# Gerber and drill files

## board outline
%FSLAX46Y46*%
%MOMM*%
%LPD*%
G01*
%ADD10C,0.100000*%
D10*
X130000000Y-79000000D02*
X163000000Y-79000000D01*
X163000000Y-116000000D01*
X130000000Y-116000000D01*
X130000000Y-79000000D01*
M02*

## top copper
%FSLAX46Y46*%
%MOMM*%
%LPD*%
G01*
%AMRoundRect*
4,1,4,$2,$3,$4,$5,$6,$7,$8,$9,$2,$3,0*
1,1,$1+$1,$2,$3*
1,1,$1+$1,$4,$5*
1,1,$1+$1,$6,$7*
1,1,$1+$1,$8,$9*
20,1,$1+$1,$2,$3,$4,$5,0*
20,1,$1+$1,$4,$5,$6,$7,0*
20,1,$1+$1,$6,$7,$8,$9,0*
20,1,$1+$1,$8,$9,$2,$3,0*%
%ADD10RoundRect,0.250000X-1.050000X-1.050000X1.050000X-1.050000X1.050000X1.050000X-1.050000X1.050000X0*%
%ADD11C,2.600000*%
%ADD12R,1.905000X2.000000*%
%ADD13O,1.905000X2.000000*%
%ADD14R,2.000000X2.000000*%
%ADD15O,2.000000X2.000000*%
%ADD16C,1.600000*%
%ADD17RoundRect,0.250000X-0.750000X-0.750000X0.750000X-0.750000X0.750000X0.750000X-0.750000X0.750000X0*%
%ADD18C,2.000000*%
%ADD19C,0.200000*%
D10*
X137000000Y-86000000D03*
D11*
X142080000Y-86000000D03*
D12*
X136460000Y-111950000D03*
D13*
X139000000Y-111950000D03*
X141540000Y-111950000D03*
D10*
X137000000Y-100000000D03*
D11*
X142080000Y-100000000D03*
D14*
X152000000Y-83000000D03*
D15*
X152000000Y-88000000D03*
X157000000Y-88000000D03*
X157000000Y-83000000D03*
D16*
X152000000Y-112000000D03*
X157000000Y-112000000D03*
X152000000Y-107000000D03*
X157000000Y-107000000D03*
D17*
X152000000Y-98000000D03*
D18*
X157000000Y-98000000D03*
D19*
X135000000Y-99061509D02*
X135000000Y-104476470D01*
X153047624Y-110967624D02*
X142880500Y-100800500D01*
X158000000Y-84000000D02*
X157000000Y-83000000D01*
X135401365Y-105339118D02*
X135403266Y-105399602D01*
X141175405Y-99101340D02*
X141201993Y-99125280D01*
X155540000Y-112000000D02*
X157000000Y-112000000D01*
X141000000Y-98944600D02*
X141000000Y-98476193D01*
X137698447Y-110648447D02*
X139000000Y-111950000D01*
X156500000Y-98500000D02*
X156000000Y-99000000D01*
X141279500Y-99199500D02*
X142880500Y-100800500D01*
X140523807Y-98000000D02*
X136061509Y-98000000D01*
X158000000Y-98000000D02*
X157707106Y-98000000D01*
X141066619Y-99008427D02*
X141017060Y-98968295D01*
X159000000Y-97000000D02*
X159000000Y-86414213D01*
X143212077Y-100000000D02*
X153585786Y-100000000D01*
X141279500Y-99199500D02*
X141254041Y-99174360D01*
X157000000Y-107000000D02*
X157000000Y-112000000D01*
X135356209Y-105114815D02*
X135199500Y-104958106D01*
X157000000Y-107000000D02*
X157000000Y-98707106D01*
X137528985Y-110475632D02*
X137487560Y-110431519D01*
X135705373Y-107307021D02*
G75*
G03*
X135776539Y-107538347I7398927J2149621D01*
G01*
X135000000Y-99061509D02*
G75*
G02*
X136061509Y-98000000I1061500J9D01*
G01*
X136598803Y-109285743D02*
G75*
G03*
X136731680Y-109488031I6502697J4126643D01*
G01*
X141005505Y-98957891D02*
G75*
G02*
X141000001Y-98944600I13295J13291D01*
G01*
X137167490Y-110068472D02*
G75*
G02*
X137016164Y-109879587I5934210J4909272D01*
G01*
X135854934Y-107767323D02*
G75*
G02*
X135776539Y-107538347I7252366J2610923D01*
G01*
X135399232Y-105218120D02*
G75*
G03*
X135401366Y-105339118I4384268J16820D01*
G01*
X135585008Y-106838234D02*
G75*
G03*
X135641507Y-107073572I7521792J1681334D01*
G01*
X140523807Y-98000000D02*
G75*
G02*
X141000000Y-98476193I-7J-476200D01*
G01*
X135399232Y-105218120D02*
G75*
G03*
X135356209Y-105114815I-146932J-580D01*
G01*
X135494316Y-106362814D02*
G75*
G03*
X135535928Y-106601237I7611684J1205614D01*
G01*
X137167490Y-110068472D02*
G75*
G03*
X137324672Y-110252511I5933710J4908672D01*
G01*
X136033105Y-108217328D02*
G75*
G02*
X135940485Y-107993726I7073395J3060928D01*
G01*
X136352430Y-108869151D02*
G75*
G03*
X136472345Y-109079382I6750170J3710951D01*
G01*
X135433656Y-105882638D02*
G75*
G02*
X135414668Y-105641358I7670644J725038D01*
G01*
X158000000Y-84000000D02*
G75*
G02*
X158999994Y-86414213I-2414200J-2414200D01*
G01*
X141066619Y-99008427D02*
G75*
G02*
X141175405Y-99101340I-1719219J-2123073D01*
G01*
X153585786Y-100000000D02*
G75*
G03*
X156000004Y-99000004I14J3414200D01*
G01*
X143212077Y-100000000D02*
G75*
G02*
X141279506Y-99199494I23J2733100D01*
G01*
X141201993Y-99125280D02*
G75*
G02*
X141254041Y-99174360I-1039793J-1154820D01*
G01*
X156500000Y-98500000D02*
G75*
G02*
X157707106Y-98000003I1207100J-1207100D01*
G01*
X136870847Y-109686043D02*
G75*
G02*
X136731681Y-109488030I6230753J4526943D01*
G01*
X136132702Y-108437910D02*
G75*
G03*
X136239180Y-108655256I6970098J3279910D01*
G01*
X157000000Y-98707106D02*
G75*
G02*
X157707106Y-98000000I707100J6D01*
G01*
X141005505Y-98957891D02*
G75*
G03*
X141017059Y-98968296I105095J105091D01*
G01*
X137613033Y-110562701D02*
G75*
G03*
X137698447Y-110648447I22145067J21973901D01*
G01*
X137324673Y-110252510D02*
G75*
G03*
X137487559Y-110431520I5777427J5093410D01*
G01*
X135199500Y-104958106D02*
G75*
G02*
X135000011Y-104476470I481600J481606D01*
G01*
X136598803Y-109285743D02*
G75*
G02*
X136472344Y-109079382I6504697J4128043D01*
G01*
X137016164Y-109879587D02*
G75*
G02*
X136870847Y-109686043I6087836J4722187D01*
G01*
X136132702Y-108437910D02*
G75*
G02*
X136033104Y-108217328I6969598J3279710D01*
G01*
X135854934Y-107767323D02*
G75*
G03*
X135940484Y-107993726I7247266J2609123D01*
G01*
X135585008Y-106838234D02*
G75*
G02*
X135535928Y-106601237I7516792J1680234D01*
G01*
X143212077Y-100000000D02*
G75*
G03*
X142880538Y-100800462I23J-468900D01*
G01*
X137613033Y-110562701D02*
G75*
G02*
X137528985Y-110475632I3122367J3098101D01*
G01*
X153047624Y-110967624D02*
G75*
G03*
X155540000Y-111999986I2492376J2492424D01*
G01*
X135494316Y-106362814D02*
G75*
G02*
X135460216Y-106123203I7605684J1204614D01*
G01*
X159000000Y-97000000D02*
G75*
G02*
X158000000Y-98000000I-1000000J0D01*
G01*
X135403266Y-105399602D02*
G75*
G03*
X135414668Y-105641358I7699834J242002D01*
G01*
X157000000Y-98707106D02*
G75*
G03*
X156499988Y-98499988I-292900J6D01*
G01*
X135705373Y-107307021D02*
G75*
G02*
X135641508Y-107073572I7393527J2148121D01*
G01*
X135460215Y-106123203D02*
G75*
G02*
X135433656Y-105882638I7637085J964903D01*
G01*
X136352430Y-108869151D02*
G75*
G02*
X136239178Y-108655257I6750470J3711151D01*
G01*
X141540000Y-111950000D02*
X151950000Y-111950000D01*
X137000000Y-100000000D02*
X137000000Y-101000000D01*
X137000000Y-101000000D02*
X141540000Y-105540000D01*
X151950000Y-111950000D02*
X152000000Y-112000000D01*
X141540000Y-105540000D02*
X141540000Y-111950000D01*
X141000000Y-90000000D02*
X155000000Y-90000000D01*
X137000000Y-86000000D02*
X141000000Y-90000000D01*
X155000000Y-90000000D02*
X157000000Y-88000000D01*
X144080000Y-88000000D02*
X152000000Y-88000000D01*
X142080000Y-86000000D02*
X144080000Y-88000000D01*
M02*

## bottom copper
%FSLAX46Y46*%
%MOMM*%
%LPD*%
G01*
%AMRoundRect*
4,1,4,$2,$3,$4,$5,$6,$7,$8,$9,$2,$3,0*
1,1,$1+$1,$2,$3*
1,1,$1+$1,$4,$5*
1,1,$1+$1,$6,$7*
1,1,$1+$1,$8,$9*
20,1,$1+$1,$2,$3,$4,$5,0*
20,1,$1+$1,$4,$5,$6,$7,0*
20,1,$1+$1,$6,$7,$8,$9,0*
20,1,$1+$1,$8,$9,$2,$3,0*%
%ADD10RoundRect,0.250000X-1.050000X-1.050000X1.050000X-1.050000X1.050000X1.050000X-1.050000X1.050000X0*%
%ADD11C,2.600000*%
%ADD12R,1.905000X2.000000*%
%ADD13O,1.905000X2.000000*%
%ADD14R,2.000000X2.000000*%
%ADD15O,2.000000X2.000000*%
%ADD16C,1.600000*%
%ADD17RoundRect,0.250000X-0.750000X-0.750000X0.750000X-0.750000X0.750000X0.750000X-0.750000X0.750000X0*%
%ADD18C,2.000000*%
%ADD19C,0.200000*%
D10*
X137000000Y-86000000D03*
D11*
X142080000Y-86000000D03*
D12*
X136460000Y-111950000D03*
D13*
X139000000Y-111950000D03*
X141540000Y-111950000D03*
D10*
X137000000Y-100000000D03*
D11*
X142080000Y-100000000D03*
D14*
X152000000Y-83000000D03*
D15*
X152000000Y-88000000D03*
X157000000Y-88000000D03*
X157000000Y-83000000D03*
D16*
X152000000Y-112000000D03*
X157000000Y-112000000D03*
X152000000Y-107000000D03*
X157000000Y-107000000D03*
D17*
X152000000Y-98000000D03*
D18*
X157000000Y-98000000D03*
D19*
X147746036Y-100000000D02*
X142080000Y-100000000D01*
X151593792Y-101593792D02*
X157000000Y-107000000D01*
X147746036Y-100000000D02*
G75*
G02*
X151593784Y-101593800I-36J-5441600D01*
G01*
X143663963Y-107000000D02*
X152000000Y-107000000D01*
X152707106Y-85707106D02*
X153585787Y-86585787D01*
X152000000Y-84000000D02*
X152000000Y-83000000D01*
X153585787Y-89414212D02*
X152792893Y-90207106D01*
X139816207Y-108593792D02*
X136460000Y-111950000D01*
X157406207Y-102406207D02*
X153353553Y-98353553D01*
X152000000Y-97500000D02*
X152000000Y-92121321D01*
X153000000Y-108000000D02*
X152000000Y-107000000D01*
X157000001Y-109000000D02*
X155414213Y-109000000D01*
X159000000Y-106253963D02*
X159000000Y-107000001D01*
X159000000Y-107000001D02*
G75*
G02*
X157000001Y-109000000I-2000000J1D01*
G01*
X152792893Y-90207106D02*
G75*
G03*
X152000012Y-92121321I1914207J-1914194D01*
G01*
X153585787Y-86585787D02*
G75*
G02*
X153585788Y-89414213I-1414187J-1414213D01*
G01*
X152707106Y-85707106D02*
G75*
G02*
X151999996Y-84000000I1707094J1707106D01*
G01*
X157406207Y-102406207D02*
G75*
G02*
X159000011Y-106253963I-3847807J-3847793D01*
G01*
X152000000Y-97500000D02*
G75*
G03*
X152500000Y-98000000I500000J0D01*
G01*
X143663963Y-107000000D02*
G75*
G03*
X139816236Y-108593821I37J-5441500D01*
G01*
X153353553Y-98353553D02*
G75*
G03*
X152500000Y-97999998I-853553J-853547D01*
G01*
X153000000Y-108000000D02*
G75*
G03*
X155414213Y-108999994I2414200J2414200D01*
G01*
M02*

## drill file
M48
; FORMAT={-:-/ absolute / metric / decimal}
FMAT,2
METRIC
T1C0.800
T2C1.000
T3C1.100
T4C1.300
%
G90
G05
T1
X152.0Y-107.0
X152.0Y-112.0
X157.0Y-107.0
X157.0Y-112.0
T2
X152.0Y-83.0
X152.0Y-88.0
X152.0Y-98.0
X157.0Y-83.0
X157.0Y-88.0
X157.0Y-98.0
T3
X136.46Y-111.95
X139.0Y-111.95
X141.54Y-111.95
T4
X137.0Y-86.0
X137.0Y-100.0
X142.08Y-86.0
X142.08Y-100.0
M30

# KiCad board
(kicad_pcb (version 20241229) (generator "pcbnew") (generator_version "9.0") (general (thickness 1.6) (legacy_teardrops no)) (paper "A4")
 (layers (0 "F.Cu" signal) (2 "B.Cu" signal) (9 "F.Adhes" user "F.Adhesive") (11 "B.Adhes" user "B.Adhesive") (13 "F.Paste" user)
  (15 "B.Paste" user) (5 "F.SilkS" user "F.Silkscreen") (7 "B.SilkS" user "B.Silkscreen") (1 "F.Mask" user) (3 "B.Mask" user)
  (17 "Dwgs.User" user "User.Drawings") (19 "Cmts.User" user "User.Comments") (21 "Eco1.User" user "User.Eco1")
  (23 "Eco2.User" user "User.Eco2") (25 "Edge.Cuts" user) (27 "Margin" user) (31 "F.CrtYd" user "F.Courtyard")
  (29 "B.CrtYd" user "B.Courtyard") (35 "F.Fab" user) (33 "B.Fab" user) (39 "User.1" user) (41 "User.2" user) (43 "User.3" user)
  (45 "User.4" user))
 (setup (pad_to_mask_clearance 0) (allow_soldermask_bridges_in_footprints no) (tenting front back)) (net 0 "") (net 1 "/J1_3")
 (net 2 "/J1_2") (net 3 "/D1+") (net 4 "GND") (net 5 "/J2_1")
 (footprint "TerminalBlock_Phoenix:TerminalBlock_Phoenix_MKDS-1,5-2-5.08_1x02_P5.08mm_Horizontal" (layer "F.Cu") (at 137 86)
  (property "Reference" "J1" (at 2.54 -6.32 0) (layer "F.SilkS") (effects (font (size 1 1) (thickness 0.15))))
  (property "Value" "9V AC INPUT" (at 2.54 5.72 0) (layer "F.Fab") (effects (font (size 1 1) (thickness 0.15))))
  (pad "1" thru_hole roundrect (at 0 0) (size 2.6 2.6) (drill 1.3) (layers "*.Cu" "*.Mask") (remove_unused_layers no)
   (roundrect_rratio 0.096154) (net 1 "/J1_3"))
  (pad "2" thru_hole circle (at 5.08 0) (size 2.6 2.6) (drill 1.3) (layers "*.Cu" "*.Mask") (remove_unused_layers no) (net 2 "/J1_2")))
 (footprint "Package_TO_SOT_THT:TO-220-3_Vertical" (layer "F.Cu") (at 136.46 111.95)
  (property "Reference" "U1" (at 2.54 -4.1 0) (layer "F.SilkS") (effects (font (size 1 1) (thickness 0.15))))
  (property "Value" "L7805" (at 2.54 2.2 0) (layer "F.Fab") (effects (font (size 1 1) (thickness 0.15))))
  (pad "1" thru_hole rect (at 0 0) (size 1.905 2) (drill 1.1) (layers "*.Cu" "*.Mask") (remove_unused_layers no) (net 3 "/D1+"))
  (pad "2" thru_hole oval (at 2.54 0) (size 1.905 2) (drill 1.1) (layers "*.Cu" "*.Mask") (remove_unused_layers no) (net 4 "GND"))
  (pad "3" thru_hole oval (at 5.08 0) (size 1.905 2) (drill 1.1) (layers "*.Cu" "*.Mask") (remove_unused_layers no) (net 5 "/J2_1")))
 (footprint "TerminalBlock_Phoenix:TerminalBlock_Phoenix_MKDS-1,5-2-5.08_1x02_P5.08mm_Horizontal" (layer "F.Cu") (at 137 100)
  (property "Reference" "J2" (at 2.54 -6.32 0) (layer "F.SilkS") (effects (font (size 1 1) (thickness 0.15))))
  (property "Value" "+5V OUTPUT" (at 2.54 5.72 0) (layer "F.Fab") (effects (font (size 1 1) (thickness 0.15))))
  (pad "1" thru_hole roundrect (at 0 0) (size 2.6 2.6) (drill 1.3) (layers "*.Cu" "*.Mask") (remove_unused_layers no)
   (roundrect_rratio 0.096154) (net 5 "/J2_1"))
  (pad "2" thru_hole circle (at 5.08 0) (size 2.6 2.6) (drill 1.3) (layers "*.Cu" "*.Mask") (remove_unused_layers no) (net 4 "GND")))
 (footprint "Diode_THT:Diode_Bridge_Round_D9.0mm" (layer "F.Cu") (at 152 83)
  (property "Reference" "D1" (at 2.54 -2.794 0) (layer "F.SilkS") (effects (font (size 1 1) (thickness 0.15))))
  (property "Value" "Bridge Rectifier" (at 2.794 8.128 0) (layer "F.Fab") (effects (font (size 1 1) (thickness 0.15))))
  (pad "1" thru_hole rect (at 0 0) (size 2 2) (drill 1) (layers "*.Cu" "*.Mask") (remove_unused_layers no) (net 3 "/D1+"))
  (pad "2" thru_hole oval (at 0 5) (size 2 2) (drill 1) (layers "*.Cu" "*.Mask") (remove_unused_layers no) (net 2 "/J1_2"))
  (pad "3" thru_hole oval (at 5 5) (size 2 2) (drill 1) (layers "*.Cu" "*.Mask") (remove_unused_layers no) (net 1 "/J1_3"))
  (pad "4" thru_hole oval (at 5 0) (size 2 2) (drill 1) (layers "*.Cu" "*.Mask") (remove_unused_layers no) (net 4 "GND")))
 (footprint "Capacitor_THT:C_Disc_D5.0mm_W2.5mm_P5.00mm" (layer "F.Cu") (at 152 112)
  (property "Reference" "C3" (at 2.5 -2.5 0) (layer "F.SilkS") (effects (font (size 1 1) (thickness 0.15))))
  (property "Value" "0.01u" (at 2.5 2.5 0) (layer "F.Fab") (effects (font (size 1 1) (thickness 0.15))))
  (pad "1" thru_hole circle (at 0 0) (size 1.6 1.6) (drill 0.8) (layers "*.Cu" "*.Mask") (remove_unused_layers no) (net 5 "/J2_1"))
  (pad "2" thru_hole circle (at 5 0) (size 1.6 1.6) (drill 0.8) (layers "*.Cu" "*.Mask") (remove_unused_layers no) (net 4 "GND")))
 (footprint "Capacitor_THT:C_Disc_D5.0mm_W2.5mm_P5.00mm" (layer "F.Cu") (at 152 107)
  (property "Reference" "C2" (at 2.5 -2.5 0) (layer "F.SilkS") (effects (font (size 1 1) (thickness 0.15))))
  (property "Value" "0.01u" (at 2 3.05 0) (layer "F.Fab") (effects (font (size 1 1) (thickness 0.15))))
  (pad "1" thru_hole circle (at 0 0) (size 1.6 1.6) (drill 0.8) (layers "*.Cu" "*.Mask") (remove_unused_layers no) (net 3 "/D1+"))
  (pad "2" thru_hole circle (at 5 0) (size 1.6 1.6) (drill 0.8) (layers "*.Cu" "*.Mask") (remove_unused_layers no) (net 4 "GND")))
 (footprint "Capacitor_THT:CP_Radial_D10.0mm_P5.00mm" (layer "F.Cu") (at 152 98)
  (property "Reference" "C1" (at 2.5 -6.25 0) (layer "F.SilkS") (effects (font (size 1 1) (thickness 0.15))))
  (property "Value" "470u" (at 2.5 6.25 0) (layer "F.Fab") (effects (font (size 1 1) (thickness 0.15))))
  (pad "1" thru_hole roundrect (at 0 0) (size 2 2) (drill 1) (layers "*.Cu" "*.Mask") (remove_unused_layers no) (roundrect_rratio 0.125)
   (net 3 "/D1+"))
  (pad "2" thru_hole circle (at 5 0) (size 2 2) (drill 1) (layers "*.Cu" "*.Mask") (remove_unused_layers no) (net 4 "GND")))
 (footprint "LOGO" (layer "F.Cu") (at 161 113 90)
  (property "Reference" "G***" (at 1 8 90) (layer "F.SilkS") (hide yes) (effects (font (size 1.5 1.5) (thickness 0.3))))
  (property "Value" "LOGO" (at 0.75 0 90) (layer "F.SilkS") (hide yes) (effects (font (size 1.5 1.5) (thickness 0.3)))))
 (gr_rect (start 130 79) (end 163 116) (stroke (width 0.1) (type solid)) (fill no) (layer "Edge.Cuts"))
 (segment (start 135 99.061509) (end 135 104.47647) (width 0.2) (layer "F.Cu") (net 4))
 (segment (start 153.047624 110.967624) (end 142.8805 100.8005) (width 0.2) (layer "F.Cu") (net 4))
 (segment (start 158 84) (end 157 83) (width 0.2) (layer "F.Cu") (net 4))
 (segment (start 135.401365 105.339118) (end 135.403266 105.399602) (width 0.2) (layer "F.Cu") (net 4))
 (segment (start 141.175405 99.10134) (end 141.201993 99.12528) (width 0.2) (layer "F.Cu") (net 4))
 (segment (start 155.54 112) (end 157 112) (width 0.2) (layer "F.Cu") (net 4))
 (segment (start 141 98.9446) (end 141 98.476193) (width 0.2) (layer "F.Cu") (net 4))
 (segment (start 137.698447 110.648447) (end 139 111.95) (width 0.2) (layer "F.Cu") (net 4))
 (segment (start 156.5 98.5) (end 156 99) (width 0.2) (layer "F.Cu") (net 4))
 (segment (start 141.2795 99.1995) (end 142.8805 100.8005) (width 0.2) (layer "F.Cu") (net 4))
 (segment (start 140.523807 98) (end 136.061509 98) (width 0.2) (layer "F.Cu") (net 4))
 (segment (start 158 98) (end 157.707106 98) (width 0.2) (layer "F.Cu") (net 4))
 (segment (start 141.066619 99.008427) (end 141.01706 98.968295) (width 0.2) (layer "F.Cu") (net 4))
 (segment (start 159 97) (end 159 86.414213) (width 0.2) (layer "F.Cu") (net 4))
 (segment (start 143.212077 100) (end 153.585786 100) (width 0.2) (layer "F.Cu") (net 4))
 (segment (start 141.2795 99.1995) (end 141.254041 99.17436) (width 0.2) (layer "F.Cu") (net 4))
 (segment (start 157 107) (end 157 112) (width 0.2) (layer "F.Cu") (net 4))
 (segment (start 135.356209 105.114815) (end 135.1995 104.958106) (width 0.2) (layer "F.Cu") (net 4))
 (segment (start 157 107) (end 157 98.707106) (width 0.2) (layer "F.Cu") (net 4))
 (segment (start 137.528985 110.475632) (end 137.48756 110.431519) (width 0.2) (layer "F.Cu") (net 4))
 (arc (start 135.705373 107.307021) (mid 135.740047 107.422963) (end 135.776538 107.538347) (width 0.2) (layer "F.Cu") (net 4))
 (arc (start 135 99.061509) (mid 135.310909 98.310909) (end 136.061509 98) (width 0.2) (layer "F.Cu") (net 4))
 (arc (start 136.598803 109.285743) (mid 136.664447 109.387408) (end 136.731681 109.48803) (width 0.2) (layer "F.Cu") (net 4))
 (arc (start 141.005505 98.957891) (mid 141.00143 98.951793) (end 141 98.9446) (width 0.2) (layer "F.Cu") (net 4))
 (arc (start 137.16749 110.068472) (mid 137.091085 109.974624) (end 137.016164 109.879587) (width 0.2) (layer "F.Cu") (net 4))
 (arc (start 135.854934 107.767323) (mid 135.814837 107.653142) (end 135.776538 107.538347) (width 0.2) (layer "F.Cu") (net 4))
 (arc (start 135.399232 105.21812) (mid 135.399881 105.278626) (end 135.401365 105.339118) (width 0.2) (layer "F.Cu") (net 4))
 (arc (start 135.585008 106.838234) (mid 135.612334 106.956124) (end 135.641508 107.073572) (width 0.2) (layer "F.Cu") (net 4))
 (arc (start 140.523807 98) (mid 140.860526 98.139473) (end 141 98.476193) (width 0.2) (layer "F.Cu") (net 4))
 (arc (start 135.399232 105.21812) (mid 135.387943 105.16221) (end 135.356209 105.114815) (width 0.2) (layer "F.Cu") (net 4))
 (arc (start 135.494316 106.362814) (mid 135.514186 106.482189) (end 135.535928 106.601237) (width 0.2) (layer "F.Cu") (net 4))
 (arc (start 137.16749 110.068472) (mid 137.245358 110.161108) (end 137.324673 110.25251) (width 0.2) (layer "F.Cu") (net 4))
 (arc (start 136.033105 108.217328) (mid 135.985917 108.10589) (end 135.940485 107.993726) (width 0.2) (layer "F.Cu") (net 4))
 (arc (start 136.35243 108.869151) (mid 136.411561 108.974737) (end 136.472344 109.079382) (width 0.2) (layer "F.Cu") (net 4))
 (arc (start 135.433656 105.882638) (mid 135.423214 105.762072) (end 135.414667 105.641358) (width 0.2) (layer "F.Cu") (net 4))
 (arc (start 158 84) (mid 158.740108 85.10765) (end 159 86.414213) (width 0.2) (layer "F.Cu") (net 4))
 (arc (start 141.066619 99.008427) (mid 141.12162 99.054171) (end 141.175405 99.10134) (width 0.2) (layer "F.Cu") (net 4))
 (arc (start 153.585786 100) (mid 154.892349 99.740108) (end 156 99) (width 0.2) (layer "F.Cu") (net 4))
 (arc (start 143.212077 100) (mid 142.166174 99.791956) (end 141.2795 99.1995) (width 0.2) (layer "F.Cu") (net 4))
 (arc (start 141.201993 99.12528) (mid 141.228299 99.14952) (end 141.254041 99.17436) (width 0.2) (layer "F.Cu") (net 4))
 (arc (start 156.5 98.5) (mid 157.053825 98.129945) (end 157.707106 98) (width 0.2) (layer "F.Cu") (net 4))
 (arc (start 136.870847 109.686043) (mid 136.800486 109.587583) (end 136.731681 109.48803) (width 0.2) (layer "F.Cu") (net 4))
 (arc (start 136.132702 108.43791) (mid 136.185087 108.547002) (end 136.239179 108.655257) (width 0.2) (layer "F.Cu") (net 4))
 (arc (start 157 98.707106) (mid 157.207106 98.207106) (end 157.707106 98) (width 0.2) (layer "F.Cu") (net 4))
 (arc (start 141.005505 98.957891) (mid 141.011146 98.963244) (end 141.01706 98.968295) (width 0.2) (layer "F.Cu") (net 4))
 (arc (start 137.613033 110.562701) (mid 137.655698 110.605615) (end 137.698447 110.648447) (width 0.2) (layer "F.Cu") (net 4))
 (arc (start 137.324673 110.25251) (mid 137.405413 110.342654) (end 137.48756 110.431519) (width 0.2) (layer "F.Cu") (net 4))
 (arc (start 135.1995 104.958106) (mid 135.051848 104.737129) (end 135 104.47647) (width 0.2) (layer "F.Cu") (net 4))
 (arc (start 136.598803 109.285743) (mid 136.534763 109.183059) (end 136.472344 109.079382) (width 0.2) (layer "F.Cu") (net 4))
 (arc (start 137.016164 109.879587) (mid 136.942745 109.783385) (end 136.870847 109.686043) (width 0.2) (layer "F.Cu") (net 4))
 (arc (start 136.132702 108.43791) (mid 136.082037 108.32801) (end 136.033105 108.217328) (width 0.2) (layer "F.Cu") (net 4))
 (arc (start 135.854934 107.767323) (mid 135.89682 107.88086) (end 135.940485 107.993726) (width 0.2) (layer "F.Cu") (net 4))
 (arc (start 135.585008 106.838234) (mid 135.559537 106.719928) (end 135.535928 106.601237) (width 0.2) (layer "F.Cu") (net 4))
 (arc (start 143.212077 100) (mid 142.77885 100.289473) (end 142.8805 100.8005) (width 0.2) (layer "F.Cu") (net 4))
 (arc (start 137.613033 110.562701) (mid 137.570709 110.519455) (end 137.528985 110.475632) (width 0.2) (layer "F.Cu") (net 4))
 (arc (start 153.047624 110.967624) (mid 154.191135 111.731694) (end 155.54 112) (width 0.2) (layer "F.Cu") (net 4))
 (arc (start 135.494316 106.362814) (mid 135.476324 106.243142) (end 135.460215 106.123203) (width 0.2) (layer "F.Cu") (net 4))
 (arc (start 159 97) (mid 158.707106 97.707106) (end 158 98) (width 0.2) (layer "F.Cu") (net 4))
 (arc (start 135.403266 105.399602) (mid 135.408017 105.520524) (end 135.414667 105.641358) (width 0.2) (layer "F.Cu") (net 4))
 (arc (start 157 98.707106) (mid 156.819192 98.436508) (end 156.5 98.5) (width 0.2) (layer "F.Cu") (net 4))
 (arc (start 135.705373 107.307021) (mid 135.672523 107.190547) (end 135.641508 107.073572) (width 0.2) (layer "F.Cu") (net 4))
 (arc (start 135.460215 106.123203) (mid 135.44599 106.003025) (end 135.433656 105.882638) (width 0.2) (layer "F.Cu") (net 4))
 (arc (start 136.35243 108.869151) (mid 136.294964 108.762648) (end 136.239179 108.655257) (width 0.2) (layer "F.Cu") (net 4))
 (segment (start 147.746036 100) (end 142.08 100) (width 0.2) (layer "B.Cu") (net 4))
 (segment (start 151.593792 101.593792) (end 157 107) (width 0.2) (layer "B.Cu") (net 4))
 (arc (start 147.746036 100) (mid 149.828426 100.414213) (end 151.593792 101.593792) (width 0.2) (layer "B.Cu") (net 4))
 (segment (start 143.663963 107) (end 152 107) (width 0.2) (layer "B.Cu") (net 3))
 (segment (start 152.707106 85.707106) (end 153.585787 86.585787) (width 0.2) (layer "B.Cu") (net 3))
 (segment (start 152 84) (end 152 83) (width 0.2) (layer "B.Cu") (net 3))
 (segment (start 153.585787 89.414212) (end 152.792893 90.207106) (width 0.2) (layer "B.Cu") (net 3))
 (segment (start 139.816207 108.593792) (end 136.46 111.95) (width 0.2) (layer "B.Cu") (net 3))
 (segment (start 157.406207 102.406207) (end 153.353553 98.353553) (width 0.2) (layer "B.Cu") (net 3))
 (segment (start 152 97.5) (end 152 92.121321) (width 0.2) (layer "B.Cu") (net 3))
 (segment (start 153 108) (end 152 107) (width 0.2) (layer "B.Cu") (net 3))
 (segment (start 157.000001 109) (end 155.414213 109) (width 0.2) (layer "B.Cu") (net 3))
 (segment (start 159 106.253963) (end 159 107.000001) (width 0.2) (layer "B.Cu") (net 3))
 (arc (start 159 107.000001) (mid 158.414213 108.414213) (end 157.000001 109) (width 0.2) (layer "B.Cu") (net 3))
 (arc (start 152.792893 90.207106) (mid 152.206066 91.085355) (end 152 92.121321) (width 0.2) (layer "B.Cu") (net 3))
 (arc (start 153.585787 86.585787) (mid 154.171573 87.999999) (end 153.585787 89.414212) (width 0.2) (layer "B.Cu") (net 3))
 (arc (start 152.707106 85.707106) (mid 152.18377 84.923879) (end 152 84) (width 0.2) (layer "B.Cu") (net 3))
 (arc (start 157.406207 102.406207) (mid 158.585786 104.171572) (end 159 106.253963) (width 0.2) (layer "B.Cu") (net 3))
 (arc (start 152 97.5) (mid 152.146446 97.853553) (end 152.5 98) (width 0.2) (layer "B.Cu") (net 3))
 (arc (start 143.663963 107) (mid 141.581572 107.414213) (end 139.816207 108.593792) (width 0.2) (layer "B.Cu") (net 3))
 (arc (start 153.353553 98.353553) (mid 152.961939 98.091885) (end 152.5 98) (width 0.2) (layer "B.Cu") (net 3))
 (arc (start 153 108) (mid 154.10765 108.740108) (end 155.414213 109) (width 0.2) (layer "B.Cu") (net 3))
 (segment (start 141.54 111.95) (end 151.95 111.95) (width 0.2) (layer "F.Cu") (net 5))
 (segment (start 137 100) (end 137 101) (width 0.2) (layer "F.Cu") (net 5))
 (segment (start 137 101) (end 141.54 105.54) (width 0.2) (layer "F.Cu") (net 5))
 (segment (start 151.95 111.95) (end 152 112) (width 0.2) (layer "F.Cu") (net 5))
 (segment (start 141.54 105.54) (end 141.54 111.95) (width 0.2) (layer "F.Cu") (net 5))
 (segment (start 141 90) (end 155 90) (width 0.2) (layer "F.Cu") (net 1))
 (segment (start 137 86) (end 141 90) (width 0.2) (layer "F.Cu") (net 1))
 (segment (start 155 90) (end 157 88) (width 0.2) (layer "F.Cu") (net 1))
 (segment (start 144.08 88) (end 152 88) (width 0.2) (layer "F.Cu") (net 2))
 (segment (start 142.08 86) (end 144.08 88) (width 0.2) (layer "F.Cu") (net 2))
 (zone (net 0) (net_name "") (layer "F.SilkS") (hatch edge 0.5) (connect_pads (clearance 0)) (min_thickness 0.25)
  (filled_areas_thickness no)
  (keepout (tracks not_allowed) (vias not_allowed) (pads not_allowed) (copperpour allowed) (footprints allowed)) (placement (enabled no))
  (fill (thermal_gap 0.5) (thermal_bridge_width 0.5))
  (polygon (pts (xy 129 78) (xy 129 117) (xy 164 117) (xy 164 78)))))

